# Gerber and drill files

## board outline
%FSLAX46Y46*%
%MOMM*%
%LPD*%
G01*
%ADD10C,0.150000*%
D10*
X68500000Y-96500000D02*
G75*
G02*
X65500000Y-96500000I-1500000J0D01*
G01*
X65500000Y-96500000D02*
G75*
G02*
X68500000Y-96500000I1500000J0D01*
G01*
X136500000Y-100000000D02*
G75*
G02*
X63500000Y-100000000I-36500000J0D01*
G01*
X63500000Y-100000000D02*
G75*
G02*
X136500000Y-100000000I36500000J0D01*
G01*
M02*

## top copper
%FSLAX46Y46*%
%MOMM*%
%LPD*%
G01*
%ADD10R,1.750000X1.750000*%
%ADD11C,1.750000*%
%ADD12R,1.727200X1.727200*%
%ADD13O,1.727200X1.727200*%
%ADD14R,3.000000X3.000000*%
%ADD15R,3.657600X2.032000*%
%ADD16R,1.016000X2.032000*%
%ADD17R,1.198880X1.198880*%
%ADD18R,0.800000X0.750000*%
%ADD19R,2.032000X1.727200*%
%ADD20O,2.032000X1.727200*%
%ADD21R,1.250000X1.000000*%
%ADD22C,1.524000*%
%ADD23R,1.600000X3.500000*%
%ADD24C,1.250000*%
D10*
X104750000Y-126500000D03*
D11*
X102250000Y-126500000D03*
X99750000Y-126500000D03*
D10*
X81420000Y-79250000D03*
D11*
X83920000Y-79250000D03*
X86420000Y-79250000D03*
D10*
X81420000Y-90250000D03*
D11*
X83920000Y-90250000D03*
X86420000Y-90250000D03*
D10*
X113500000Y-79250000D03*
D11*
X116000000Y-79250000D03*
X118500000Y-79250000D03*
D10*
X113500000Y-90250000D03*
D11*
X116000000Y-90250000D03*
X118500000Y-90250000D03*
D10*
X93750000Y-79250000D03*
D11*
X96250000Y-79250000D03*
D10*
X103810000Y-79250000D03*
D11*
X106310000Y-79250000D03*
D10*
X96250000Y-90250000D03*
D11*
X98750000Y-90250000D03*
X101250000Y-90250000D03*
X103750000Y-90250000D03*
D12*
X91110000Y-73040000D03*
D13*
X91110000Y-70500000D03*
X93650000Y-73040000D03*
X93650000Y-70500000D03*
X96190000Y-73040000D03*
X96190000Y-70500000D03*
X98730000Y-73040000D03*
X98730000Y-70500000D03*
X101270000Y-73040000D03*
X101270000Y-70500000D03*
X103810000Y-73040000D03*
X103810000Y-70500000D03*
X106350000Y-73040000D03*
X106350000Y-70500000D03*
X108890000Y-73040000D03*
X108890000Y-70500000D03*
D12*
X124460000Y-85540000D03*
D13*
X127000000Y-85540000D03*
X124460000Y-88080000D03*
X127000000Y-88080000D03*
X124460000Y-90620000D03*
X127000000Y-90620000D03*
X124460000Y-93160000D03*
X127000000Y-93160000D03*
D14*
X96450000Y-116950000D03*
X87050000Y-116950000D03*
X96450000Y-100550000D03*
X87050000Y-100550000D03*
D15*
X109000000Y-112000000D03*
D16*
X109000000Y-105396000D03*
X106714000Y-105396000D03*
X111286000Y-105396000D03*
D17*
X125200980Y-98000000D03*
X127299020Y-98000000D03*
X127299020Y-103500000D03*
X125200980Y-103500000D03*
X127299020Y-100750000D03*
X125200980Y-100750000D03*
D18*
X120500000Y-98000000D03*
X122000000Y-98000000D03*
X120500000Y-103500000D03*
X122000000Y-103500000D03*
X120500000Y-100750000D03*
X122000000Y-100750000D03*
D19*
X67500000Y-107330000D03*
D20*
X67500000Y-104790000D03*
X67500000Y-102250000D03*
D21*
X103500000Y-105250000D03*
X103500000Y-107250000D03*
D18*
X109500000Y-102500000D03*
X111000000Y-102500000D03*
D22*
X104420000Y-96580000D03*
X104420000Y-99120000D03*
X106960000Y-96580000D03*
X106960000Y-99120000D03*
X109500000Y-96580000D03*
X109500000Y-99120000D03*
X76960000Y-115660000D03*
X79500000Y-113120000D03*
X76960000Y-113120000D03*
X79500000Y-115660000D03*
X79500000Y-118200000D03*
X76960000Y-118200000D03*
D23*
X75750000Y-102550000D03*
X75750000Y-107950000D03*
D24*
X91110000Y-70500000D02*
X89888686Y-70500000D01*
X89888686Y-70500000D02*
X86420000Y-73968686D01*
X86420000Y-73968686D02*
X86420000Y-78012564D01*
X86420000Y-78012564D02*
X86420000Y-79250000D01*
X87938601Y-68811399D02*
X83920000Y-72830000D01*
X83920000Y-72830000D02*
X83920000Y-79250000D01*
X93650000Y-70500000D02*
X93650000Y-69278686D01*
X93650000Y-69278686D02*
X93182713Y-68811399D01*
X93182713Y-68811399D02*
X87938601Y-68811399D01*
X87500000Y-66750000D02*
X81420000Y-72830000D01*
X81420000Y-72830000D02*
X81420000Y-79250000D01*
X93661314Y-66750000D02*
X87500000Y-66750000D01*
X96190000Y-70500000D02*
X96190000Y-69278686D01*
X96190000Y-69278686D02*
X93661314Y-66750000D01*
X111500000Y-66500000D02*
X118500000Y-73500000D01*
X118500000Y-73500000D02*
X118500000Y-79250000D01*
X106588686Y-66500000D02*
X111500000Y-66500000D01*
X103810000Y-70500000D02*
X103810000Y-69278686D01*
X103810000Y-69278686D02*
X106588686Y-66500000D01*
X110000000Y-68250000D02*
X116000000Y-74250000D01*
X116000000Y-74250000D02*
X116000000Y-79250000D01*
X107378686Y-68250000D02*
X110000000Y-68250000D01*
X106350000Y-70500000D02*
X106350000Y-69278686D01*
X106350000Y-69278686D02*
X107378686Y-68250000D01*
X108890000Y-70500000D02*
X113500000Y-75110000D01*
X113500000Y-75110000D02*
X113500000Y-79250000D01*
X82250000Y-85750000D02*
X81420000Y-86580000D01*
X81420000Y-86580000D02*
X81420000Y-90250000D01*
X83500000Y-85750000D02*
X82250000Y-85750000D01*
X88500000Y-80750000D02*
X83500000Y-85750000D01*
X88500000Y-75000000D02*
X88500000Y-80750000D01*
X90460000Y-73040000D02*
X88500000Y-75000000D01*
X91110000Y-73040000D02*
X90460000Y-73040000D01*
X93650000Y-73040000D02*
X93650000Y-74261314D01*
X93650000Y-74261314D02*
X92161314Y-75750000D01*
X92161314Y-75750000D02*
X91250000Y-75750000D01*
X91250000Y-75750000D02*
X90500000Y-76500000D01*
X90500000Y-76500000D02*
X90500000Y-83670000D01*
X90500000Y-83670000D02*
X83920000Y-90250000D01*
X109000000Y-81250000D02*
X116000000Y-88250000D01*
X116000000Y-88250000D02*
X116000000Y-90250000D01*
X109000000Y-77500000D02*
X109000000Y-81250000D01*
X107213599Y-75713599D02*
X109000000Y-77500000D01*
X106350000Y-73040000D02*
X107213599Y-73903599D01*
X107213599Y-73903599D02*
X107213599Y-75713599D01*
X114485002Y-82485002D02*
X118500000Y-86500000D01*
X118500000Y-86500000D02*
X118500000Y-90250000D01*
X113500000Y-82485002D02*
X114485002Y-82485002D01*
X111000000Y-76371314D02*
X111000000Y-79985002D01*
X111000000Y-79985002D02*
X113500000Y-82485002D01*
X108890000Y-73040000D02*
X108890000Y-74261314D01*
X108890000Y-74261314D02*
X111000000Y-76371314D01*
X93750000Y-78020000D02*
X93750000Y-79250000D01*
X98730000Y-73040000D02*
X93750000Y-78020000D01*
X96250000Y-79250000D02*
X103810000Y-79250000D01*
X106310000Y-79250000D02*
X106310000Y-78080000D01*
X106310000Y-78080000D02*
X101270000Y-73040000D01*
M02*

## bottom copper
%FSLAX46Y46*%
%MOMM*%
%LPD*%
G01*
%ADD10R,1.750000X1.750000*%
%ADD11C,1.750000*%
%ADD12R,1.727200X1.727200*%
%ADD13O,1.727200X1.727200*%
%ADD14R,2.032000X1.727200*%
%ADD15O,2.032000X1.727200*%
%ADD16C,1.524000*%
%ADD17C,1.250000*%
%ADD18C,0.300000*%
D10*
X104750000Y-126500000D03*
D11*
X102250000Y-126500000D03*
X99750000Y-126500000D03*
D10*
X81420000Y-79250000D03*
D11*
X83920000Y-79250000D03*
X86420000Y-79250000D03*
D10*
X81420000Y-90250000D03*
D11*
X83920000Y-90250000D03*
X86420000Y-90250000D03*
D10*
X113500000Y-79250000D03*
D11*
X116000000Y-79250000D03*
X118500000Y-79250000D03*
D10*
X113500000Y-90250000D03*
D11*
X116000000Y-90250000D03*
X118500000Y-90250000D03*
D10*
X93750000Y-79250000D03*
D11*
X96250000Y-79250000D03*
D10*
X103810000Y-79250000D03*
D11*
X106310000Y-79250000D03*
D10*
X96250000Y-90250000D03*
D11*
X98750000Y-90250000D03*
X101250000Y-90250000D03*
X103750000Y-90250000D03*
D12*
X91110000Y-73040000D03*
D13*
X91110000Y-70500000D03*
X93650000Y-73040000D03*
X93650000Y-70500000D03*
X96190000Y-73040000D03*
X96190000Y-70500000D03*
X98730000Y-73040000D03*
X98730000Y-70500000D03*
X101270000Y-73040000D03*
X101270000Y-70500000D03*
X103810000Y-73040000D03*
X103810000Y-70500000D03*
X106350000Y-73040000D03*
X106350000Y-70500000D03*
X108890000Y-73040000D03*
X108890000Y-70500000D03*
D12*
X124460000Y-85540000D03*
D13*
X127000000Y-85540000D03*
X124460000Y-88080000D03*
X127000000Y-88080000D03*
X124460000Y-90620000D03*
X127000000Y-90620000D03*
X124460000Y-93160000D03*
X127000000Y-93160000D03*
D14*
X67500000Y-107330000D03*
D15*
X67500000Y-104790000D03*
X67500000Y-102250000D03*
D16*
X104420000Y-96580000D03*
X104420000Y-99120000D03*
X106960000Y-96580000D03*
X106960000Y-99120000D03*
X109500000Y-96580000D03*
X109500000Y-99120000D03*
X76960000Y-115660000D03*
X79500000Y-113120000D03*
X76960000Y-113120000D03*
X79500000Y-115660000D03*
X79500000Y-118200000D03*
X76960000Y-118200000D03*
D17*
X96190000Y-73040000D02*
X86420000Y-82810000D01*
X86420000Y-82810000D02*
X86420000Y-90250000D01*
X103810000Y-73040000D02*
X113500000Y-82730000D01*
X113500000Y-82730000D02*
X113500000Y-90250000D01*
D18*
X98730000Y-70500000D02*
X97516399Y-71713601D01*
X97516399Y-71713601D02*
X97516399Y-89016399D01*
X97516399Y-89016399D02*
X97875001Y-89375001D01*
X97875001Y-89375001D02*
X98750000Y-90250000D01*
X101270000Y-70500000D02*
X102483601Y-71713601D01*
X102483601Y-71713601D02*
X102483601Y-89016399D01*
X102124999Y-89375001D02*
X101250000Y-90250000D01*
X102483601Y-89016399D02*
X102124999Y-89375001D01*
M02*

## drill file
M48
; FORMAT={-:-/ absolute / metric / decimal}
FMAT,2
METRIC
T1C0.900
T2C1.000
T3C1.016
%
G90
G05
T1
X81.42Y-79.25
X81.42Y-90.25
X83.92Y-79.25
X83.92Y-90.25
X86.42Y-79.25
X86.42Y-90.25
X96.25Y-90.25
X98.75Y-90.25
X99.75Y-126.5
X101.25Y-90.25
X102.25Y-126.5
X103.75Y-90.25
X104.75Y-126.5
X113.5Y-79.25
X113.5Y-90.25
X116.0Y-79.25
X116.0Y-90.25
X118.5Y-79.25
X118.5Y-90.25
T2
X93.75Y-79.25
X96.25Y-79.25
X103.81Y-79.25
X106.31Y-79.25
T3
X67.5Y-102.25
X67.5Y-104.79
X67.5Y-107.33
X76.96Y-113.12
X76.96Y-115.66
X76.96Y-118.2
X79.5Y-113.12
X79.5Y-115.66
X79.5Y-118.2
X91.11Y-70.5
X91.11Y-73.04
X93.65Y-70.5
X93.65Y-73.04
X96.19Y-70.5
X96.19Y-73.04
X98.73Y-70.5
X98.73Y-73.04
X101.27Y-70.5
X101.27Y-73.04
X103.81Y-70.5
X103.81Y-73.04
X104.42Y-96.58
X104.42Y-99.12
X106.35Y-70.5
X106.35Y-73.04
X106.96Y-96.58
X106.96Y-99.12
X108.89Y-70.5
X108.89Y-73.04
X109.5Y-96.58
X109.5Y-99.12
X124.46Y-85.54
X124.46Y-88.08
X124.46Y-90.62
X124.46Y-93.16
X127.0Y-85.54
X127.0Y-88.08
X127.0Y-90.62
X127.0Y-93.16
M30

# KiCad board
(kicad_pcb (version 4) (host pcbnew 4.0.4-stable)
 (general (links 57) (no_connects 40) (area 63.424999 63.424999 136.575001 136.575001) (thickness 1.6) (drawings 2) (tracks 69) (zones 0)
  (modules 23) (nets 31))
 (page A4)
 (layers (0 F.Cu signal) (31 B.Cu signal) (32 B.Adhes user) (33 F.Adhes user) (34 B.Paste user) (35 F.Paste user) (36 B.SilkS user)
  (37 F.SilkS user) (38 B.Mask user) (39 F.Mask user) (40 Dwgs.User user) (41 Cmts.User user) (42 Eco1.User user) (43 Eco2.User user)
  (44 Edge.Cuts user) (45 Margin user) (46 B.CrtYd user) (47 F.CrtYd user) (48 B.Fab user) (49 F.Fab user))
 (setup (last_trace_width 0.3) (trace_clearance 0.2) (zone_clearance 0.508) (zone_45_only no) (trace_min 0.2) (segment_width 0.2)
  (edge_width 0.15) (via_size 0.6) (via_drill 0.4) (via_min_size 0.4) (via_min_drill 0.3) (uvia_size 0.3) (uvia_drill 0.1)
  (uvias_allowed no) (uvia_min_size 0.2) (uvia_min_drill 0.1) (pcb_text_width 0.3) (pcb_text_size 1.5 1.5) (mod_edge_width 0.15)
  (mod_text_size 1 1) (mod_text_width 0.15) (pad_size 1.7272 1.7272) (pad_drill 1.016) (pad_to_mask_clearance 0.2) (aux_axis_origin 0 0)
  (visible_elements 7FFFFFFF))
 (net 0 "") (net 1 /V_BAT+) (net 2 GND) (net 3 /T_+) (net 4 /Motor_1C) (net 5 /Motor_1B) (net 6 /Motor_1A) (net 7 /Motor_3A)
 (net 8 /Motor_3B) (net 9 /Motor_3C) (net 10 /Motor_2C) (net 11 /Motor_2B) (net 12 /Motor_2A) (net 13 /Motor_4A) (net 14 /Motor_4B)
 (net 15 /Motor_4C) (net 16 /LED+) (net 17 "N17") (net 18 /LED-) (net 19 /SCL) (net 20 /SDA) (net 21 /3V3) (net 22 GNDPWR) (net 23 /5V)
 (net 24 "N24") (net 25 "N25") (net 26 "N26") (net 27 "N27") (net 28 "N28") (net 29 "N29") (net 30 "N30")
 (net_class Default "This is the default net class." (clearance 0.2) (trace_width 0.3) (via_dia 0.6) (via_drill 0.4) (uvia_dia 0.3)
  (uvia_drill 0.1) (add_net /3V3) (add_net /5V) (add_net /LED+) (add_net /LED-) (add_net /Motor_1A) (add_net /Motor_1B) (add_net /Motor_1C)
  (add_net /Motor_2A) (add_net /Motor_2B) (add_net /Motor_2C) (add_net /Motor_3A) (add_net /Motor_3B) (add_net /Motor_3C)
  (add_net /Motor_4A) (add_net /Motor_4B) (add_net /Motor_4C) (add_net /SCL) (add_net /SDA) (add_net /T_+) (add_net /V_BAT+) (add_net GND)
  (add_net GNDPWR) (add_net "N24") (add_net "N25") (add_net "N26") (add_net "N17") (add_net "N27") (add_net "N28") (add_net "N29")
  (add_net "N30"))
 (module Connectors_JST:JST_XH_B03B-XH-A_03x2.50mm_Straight (layer F.Cu) (at 104.75 126.5 180)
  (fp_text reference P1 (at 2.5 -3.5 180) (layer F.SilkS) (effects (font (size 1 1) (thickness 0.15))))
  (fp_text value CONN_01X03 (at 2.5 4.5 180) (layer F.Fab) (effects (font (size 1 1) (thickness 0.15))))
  (pad 1 thru_hole rect (at 0 0 180) (size 1.75 1.75) (drill 0.9) (layers *.Cu *.Mask) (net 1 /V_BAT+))
  (pad 2 thru_hole circle (at 2.5 0 180) (size 1.75 1.75) (drill 0.9) (layers *.Cu *.Mask) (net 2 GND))
  (pad 3 thru_hole circle (at 5 0 180) (size 1.75 1.75) (drill 0.9) (layers *.Cu *.Mask) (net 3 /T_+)))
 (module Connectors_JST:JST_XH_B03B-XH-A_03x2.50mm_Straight (layer F.Cu) (at 81.42 79.25)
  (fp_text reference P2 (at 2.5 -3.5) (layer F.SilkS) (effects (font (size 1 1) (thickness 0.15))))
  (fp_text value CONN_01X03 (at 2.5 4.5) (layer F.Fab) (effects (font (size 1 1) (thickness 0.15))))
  (pad 1 thru_hole rect (at 0 0) (size 1.75 1.75) (drill 0.9) (layers *.Cu *.Mask) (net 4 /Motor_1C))
  (pad 2 thru_hole circle (at 2.5 0) (size 1.75 1.75) (drill 0.9) (layers *.Cu *.Mask) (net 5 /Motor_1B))
  (pad 3 thru_hole circle (at 5 0) (size 1.75 1.75) (drill 0.9) (layers *.Cu *.Mask) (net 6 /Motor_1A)))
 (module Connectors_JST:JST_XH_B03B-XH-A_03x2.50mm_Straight (layer F.Cu) (at 81.42 90.25)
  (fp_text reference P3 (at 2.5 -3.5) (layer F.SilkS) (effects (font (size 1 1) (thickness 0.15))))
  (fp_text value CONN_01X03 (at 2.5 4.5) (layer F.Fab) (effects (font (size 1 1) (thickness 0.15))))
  (pad 1 thru_hole rect (at 0 0) (size 1.75 1.75) (drill 0.9) (layers *.Cu *.Mask) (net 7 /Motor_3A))
  (pad 2 thru_hole circle (at 2.5 0) (size 1.75 1.75) (drill 0.9) (layers *.Cu *.Mask) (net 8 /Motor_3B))
  (pad 3 thru_hole circle (at 5 0) (size 1.75 1.75) (drill 0.9) (layers *.Cu *.Mask) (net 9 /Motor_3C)))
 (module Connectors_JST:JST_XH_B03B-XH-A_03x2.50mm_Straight (layer F.Cu) (at 113.5 79.25)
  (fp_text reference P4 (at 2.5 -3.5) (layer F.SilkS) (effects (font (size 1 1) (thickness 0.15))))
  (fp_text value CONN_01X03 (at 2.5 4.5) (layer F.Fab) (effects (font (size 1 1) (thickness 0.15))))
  (pad 1 thru_hole rect (at 0 0) (size 1.75 1.75) (drill 0.9) (layers *.Cu *.Mask) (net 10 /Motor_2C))
  (pad 2 thru_hole circle (at 2.5 0) (size 1.75 1.75) (drill 0.9) (layers *.Cu *.Mask) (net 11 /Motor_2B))
  (pad 3 thru_hole circle (at 5 0) (size 1.75 1.75) (drill 0.9) (layers *.Cu *.Mask) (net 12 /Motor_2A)))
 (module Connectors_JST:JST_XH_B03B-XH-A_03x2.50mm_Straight (layer F.Cu) (at 113.5 90.25)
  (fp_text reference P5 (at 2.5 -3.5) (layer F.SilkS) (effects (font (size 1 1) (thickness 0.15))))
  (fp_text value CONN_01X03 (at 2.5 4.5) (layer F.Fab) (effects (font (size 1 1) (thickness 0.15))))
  (pad 1 thru_hole rect (at 0 0) (size 1.75 1.75) (drill 0.9) (layers *.Cu *.Mask) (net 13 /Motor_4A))
  (pad 2 thru_hole circle (at 2.5 0) (size 1.75 1.75) (drill 0.9) (layers *.Cu *.Mask) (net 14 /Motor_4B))
  (pad 3 thru_hole circle (at 5 0) (size 1.75 1.75) (drill 0.9) (layers *.Cu *.Mask) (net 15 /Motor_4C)))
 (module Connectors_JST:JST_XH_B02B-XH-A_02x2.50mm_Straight (layer F.Cu) (at 93.75 79.25)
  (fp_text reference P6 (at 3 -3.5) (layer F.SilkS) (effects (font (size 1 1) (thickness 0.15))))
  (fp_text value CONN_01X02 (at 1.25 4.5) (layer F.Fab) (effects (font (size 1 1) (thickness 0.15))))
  (pad 1 thru_hole rect (at 0 0) (size 1.75 1.75) (drill 1) (layers *.Cu *.Mask) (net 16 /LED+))
  (pad 2 thru_hole circle (at 2.5 0) (size 1.75 1.75) (drill 1) (layers *.Cu *.Mask) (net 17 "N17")))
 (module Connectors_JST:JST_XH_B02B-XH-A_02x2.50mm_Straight (layer F.Cu) (at 103.81 79.25)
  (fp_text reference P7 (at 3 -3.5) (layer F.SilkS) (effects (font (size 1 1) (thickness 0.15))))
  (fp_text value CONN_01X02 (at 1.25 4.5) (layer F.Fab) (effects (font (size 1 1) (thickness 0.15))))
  (pad 1 thru_hole rect (at 0 0) (size 1.75 1.75) (drill 1) (layers *.Cu *.Mask) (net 17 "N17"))
  (pad 2 thru_hole circle (at 2.5 0) (size 1.75 1.75) (drill 1) (layers *.Cu *.Mask) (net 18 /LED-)))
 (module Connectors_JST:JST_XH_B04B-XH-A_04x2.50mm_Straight (layer F.Cu) (at 96.25 90.25)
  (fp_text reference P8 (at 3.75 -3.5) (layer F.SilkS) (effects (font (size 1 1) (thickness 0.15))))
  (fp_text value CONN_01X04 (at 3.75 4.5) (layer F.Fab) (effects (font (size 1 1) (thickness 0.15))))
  (pad 1 thru_hole rect (at 0 0) (size 1.75 1.75) (drill 0.9) (layers *.Cu *.Mask) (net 2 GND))
  (pad 2 thru_hole circle (at 2.5 0) (size 1.75 1.75) (drill 0.9) (layers *.Cu *.Mask) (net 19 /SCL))
  (pad 3 thru_hole circle (at 5 0) (size 1.75 1.75) (drill 0.9) (layers *.Cu *.Mask) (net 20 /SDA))
  (pad 4 thru_hole circle (at 7.5 0) (size 1.75 1.75) (drill 0.9) (layers *.Cu *.Mask) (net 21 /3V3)))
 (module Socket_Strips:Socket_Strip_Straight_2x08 (layer B.Cu) (at 91.11 73.04)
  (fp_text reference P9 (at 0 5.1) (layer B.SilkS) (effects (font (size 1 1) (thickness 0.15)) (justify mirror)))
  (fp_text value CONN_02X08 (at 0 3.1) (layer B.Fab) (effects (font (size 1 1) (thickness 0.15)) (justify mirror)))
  (pad 1 thru_hole rect (at 0 0) (size 1.7272 1.7272) (drill 1.016) (layers *.Cu *.Mask B.SilkS) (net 7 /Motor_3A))
  (pad 2 thru_hole oval (at 0 -2.54) (size 1.7272 1.7272) (drill 1.016) (layers *.Cu *.Mask B.SilkS) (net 6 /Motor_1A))
  (pad 3 thru_hole oval (at 2.54 0) (size 1.7272 1.7272) (drill 1.016) (layers *.Cu *.Mask B.SilkS) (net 8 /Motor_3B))
  (pad 4 thru_hole oval (at 2.54 -2.54) (size 1.7272 1.7272) (drill 1.016) (layers *.Cu *.Mask B.SilkS) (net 5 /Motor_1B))
  (pad 5 thru_hole oval (at 5.08 0) (size 1.7272 1.7272) (drill 1.016) (layers *.Cu *.Mask B.SilkS) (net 9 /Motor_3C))
  (pad 6 thru_hole oval (at 5.08 -2.54) (size 1.7272 1.7272) (drill 1.016) (layers *.Cu *.Mask B.SilkS) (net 4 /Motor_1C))
  (pad 7 thru_hole oval (at 7.62 0) (size 1.7272 1.7272) (drill 1.016) (layers *.Cu *.Mask B.SilkS) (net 16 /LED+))
  (pad 8 thru_hole oval (at 7.62 -2.54) (size 1.7272 1.7272) (drill 1.016) (layers *.Cu *.Mask B.SilkS) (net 19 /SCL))
  (pad 9 thru_hole oval (at 10.16 0) (size 1.7272 1.7272) (drill 1.016) (layers *.Cu *.Mask B.SilkS) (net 18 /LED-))
  (pad 10 thru_hole oval (at 10.16 -2.54) (size 1.7272 1.7272) (drill 1.016) (layers *.Cu *.Mask B.SilkS) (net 20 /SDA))
  (pad 11 thru_hole oval (at 12.7 0) (size 1.7272 1.7272) (drill 1.016) (layers *.Cu *.Mask B.SilkS) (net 13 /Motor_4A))
  (pad 12 thru_hole oval (at 12.7 -2.54) (size 1.7272 1.7272) (drill 1.016) (layers *.Cu *.Mask B.SilkS) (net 12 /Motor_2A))
  (pad 13 thru_hole oval (at 15.24 0) (size 1.7272 1.7272) (drill 1.016) (layers *.Cu *.Mask B.SilkS) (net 14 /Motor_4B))
  (pad 14 thru_hole oval (at 15.24 -2.54) (size 1.7272 1.7272) (drill 1.016) (layers *.Cu *.Mask B.SilkS) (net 11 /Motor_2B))
  (pad 15 thru_hole oval (at 17.78 0) (size 1.7272 1.7272) (drill 1.016) (layers *.Cu *.Mask B.SilkS) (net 15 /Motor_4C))
  (pad 16 thru_hole oval (at 17.78 -2.54) (size 1.7272 1.7272) (drill 1.016) (layers *.Cu *.Mask B.SilkS) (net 10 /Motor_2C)))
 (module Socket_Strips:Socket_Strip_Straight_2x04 (layer B.Cu) (at 124.46 85.54 270)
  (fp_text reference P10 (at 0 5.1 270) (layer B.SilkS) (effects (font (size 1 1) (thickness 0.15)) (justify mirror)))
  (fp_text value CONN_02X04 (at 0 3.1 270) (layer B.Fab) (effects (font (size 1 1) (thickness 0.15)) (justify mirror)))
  (pad 1 thru_hole rect (at 0 0 270) (size 1.7272 1.7272) (drill 1.016) (layers *.Cu *.Mask B.SilkS) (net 1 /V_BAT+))
  (pad 2 thru_hole oval (at 0 -2.54 270) (size 1.7272 1.7272) (drill 1.016) (layers *.Cu *.Mask B.SilkS) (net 1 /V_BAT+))
  (pad 3 thru_hole oval (at 2.54 0 270) (size 1.7272 1.7272) (drill 1.016) (layers *.Cu *.Mask B.SilkS) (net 1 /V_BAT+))
  (pad 4 thru_hole oval (at 2.54 -2.54 270) (size 1.7272 1.7272) (drill 1.016) (layers *.Cu *.Mask B.SilkS) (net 1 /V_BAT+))
  (pad 5 thru_hole oval (at 5.08 0 270) (size 1.7272 1.7272) (drill 1.016) (layers *.Cu *.Mask B.SilkS) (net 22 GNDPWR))
  (pad 6 thru_hole oval (at 5.08 -2.54 270) (size 1.7272 1.7272) (drill 1.016) (layers *.Cu *.Mask B.SilkS) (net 22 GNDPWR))
  (pad 7 thru_hole oval (at 7.62 0 270) (size 1.7272 1.7272) (drill 1.016) (layers *.Cu *.Mask B.SilkS) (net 22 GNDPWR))
  (pad 8 thru_hole oval (at 7.62 -2.54 270) (size 1.7272 1.7272) (drill 1.016) (layers *.Cu *.Mask B.SilkS) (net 22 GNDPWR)))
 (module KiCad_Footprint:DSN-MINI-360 (layer F.Cu) (at 91.75 108.75 270)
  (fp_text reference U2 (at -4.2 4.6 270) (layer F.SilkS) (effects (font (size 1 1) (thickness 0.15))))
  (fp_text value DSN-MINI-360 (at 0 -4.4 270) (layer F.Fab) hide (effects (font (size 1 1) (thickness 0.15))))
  (pad 1 smd rect (at 8.2 -4.7 270) (size 3 3) (layers F.Cu F.Paste F.Mask) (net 1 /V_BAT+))
  (pad 2 smd rect (at 8.2 4.7 270) (size 3 3) (layers F.Cu F.Paste F.Mask) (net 22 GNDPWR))
  (pad 3 smd rect (at -8.2 -4.7 270) (size 3 3) (layers F.Cu F.Paste F.Mask) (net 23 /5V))
  (pad 4 smd rect (at -8.2 4.7 270) (size 3 3) (layers F.Cu F.Paste F.Mask) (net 2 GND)))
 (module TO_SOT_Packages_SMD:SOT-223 (layer F.Cu) (at 109 108.698 180)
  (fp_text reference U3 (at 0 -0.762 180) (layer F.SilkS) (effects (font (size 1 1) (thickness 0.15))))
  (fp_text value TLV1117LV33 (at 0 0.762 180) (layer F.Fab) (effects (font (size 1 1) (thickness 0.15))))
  (pad 4 smd rect (at 0 -3.302 180) (size 3.6576 2.032) (layers F.Cu F.Paste F.Mask) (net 21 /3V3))
  (pad 2 smd rect (at 0 3.302 180) (size 1.016 2.032) (layers F.Cu F.Paste F.Mask) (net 21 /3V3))
  (pad 3 smd rect (at 2.286 3.302 180) (size 1.016 2.032) (layers F.Cu F.Paste F.Mask) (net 23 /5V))
  (pad 1 smd rect (at -2.286 3.302 180) (size 1.016 2.032) (layers F.Cu F.Paste F.Mask) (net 2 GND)))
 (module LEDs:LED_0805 (layer F.Cu) (at 126.25 98 180)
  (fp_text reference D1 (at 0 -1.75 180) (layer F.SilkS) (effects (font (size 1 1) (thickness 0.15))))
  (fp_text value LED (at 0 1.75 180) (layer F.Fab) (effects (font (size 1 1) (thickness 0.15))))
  (pad 2 smd rect (at 1.04902 0) (size 1.19888 1.19888) (layers F.Cu F.Paste F.Mask) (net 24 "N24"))
  (pad 1 smd rect (at -1.04902 0) (size 1.19888 1.19888) (layers F.Cu F.Paste F.Mask) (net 2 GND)))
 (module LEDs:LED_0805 (layer F.Cu) (at 126.25 103.5)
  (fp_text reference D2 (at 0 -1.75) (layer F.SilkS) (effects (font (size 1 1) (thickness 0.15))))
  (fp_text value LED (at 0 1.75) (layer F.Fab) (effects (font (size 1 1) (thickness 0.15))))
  (pad 2 smd rect (at 1.04902 0 180) (size 1.19888 1.19888) (layers F.Cu F.Paste F.Mask) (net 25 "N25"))
  (pad 1 smd rect (at -1.04902 0 180) (size 1.19888 1.19888) (layers F.Cu F.Paste F.Mask) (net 2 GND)))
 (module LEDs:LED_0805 (layer F.Cu) (at 126.25 100.75)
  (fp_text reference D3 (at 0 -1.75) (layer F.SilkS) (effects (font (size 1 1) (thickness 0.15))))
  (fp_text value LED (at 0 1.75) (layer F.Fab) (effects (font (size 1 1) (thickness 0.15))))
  (pad 2 smd rect (at 1.04902 0 180) (size 1.19888 1.19888) (layers F.Cu F.Paste F.Mask) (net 21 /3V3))
  (pad 1 smd rect (at -1.04902 0 180) (size 1.19888 1.19888) (layers F.Cu F.Paste F.Mask) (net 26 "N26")))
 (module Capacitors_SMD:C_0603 (layer F.Cu) (at 121.25 98)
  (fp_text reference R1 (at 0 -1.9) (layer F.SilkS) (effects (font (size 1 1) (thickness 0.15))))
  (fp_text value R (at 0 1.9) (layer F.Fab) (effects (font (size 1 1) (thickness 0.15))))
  (pad 1 smd rect (at -0.75 0) (size 0.8 0.75) (layers F.Cu F.Paste F.Mask) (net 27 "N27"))
  (pad 2 smd rect (at 0.75 0) (size 0.8 0.75) (layers F.Cu F.Paste F.Mask) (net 24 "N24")))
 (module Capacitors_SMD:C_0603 (layer F.Cu) (at 121.25 103.5)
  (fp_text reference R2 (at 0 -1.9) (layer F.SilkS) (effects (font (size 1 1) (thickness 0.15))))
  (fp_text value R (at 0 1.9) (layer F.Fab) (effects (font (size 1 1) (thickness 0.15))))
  (pad 1 smd rect (at -0.75 0) (size 0.8 0.75) (layers F.Cu F.Paste F.Mask) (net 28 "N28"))
  (pad 2 smd rect (at 0.75 0) (size 0.8 0.75) (layers F.Cu F.Paste F.Mask) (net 25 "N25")))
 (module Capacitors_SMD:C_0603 (layer F.Cu) (at 121.25 100.75)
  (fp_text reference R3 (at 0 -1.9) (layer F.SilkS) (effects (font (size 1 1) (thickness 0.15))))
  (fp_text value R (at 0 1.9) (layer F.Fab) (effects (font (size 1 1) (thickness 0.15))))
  (pad 1 smd rect (at -0.75 0) (size 0.8 0.75) (layers F.Cu F.Paste F.Mask) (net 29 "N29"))
  (pad 2 smd rect (at 0.75 0) (size 0.8 0.75) (layers F.Cu F.Paste F.Mask) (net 26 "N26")))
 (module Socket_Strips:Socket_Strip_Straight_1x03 (layer B.Cu) (at 67.5 107.33 90)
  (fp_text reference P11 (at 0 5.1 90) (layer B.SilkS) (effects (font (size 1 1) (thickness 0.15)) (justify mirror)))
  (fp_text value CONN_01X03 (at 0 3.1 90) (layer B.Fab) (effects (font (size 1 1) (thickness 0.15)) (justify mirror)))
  (pad 1 thru_hole rect (at 0 0 90) (size 1.7272 2.032) (drill 1.016) (layers *.Cu *.Mask B.SilkS) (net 2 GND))
  (pad 2 thru_hole oval (at 2.54 0 90) (size 1.7272 2.032) (drill 1.016) (layers *.Cu *.Mask B.SilkS))
  (pad 3 thru_hole oval (at 5.08 0 90) (size 1.7272 2.032) (drill 1.016) (layers *.Cu *.Mask B.SilkS) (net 23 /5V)))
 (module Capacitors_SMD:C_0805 (layer F.Cu) (at 103.5 106.25 270)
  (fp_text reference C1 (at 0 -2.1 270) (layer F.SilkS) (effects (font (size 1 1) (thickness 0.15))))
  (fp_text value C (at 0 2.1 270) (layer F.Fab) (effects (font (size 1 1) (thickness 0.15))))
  (pad 1 smd rect (at -1 0 270) (size 1 1.25) (layers F.Cu F.Paste F.Mask) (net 23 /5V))
  (pad 2 smd rect (at 1 0 270) (size 1 1.25) (layers F.Cu F.Paste F.Mask) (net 2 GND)))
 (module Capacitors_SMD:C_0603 (layer F.Cu) (at 110.25 102.5)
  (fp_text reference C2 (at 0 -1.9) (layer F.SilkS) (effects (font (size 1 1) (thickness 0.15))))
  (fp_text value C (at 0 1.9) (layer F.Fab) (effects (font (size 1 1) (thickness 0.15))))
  (pad 1 smd rect (at -0.75 0) (size 0.8 0.75) (layers F.Cu F.Paste F.Mask) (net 21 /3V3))
  (pad 2 smd rect (at 0.75 0) (size 0.8 0.75) (layers F.Cu F.Paste F.Mask) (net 2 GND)))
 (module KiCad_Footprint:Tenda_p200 (layer B.Cu) (at 93.32 100)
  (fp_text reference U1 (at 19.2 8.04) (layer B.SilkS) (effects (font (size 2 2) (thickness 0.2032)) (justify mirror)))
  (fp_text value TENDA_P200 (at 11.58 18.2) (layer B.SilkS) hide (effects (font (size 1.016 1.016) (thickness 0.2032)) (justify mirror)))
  (pad 3V3 thru_hole circle (at 11.1 -3.42) (size 1.524 1.524) (drill 1.016) (layers *.Cu *.Mask B.SilkS) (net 21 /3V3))
  (pad 3V3 thru_hole circle (at 11.1 -0.88) (size 1.524 1.524) (drill 1.016) (layers *.Cu *.Mask B.SilkS) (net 21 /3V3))
  (pad C thru_hole circle (at 13.64 -3.42) (size 1.524 1.524) (drill 1.016) (layers *.Cu *.Mask B.SilkS) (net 28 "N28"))
  (pad P thru_hole circle (at 13.64 -0.88) (size 1.524 1.524) (drill 1.016) (layers *.Cu *.Mask B.SilkS) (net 27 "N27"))
  (pad E thru_hole circle (at 16.18 -3.42) (size 1.524 1.524) (drill 1.016) (layers *.Cu *.Mask B.SilkS) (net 29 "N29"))
  (pad GND thru_hole circle (at 16.18 -0.88) (size 1.524 1.524) (drill 1.016) (layers *.Cu *.Mask B.SilkS) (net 2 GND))
  (pad NC thru_hole circle (at -16.36 15.66 270) (size 1.524 1.524) (drill 1.016) (layers *.Cu *.Mask B.SilkS) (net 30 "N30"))
  (pad T_+ thru_hole circle (at -13.82 13.12 270) (size 1.524 1.524) (drill 1.016) (layers *.Cu *.Mask B.SilkS) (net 3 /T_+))
  (pad T_+ thru_hole circle (at -16.36 13.12 270) (size 1.524 1.524) (drill 1.016) (layers *.Cu *.Mask B.SilkS) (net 3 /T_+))
  (pad NC thru_hole circle (at -13.82 15.66 270) (size 1.524 1.524) (drill 1.016) (layers *.Cu *.Mask B.SilkS) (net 30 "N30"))
  (pad T_- thru_hole circle (at -13.82 18.2 270) (size 1.524 1.524) (drill 1.016) (layers *.Cu *.Mask B.SilkS) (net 22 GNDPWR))
  (pad T_- thru_hole circle (at -16.36 18.2 270) (size 1.524 1.524) (drill 1.016) (layers *.Cu *.Mask B.SilkS) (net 22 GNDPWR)))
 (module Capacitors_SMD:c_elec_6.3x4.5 (layer F.Cu) (at 75.75 105.25 270)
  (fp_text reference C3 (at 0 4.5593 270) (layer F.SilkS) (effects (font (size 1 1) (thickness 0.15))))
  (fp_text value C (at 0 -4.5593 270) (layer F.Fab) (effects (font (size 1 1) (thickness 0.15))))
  (pad 1 smd rect (at -2.7 0 90) (size 3.5 1.6) (layers F.Cu F.Paste F.Mask) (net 23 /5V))
  (pad 2 smd rect (at 2.7 0 90) (size 3.5 1.6) (layers F.Cu F.Paste F.Mask) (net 2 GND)))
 (gr_circle (center 67 96.5) (end 67 98) (layer Edge.Cuts) (width 0.15))
 (gr_circle (center 100 100) (end 100 136.5) (layer Edge.Cuts) (width 0.15))
 (segment (start 91.11 70.5) (end 89.888686 70.5) (width 1.25) (layer F.Cu) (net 6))
 (segment (start 89.888686 70.5) (end 86.42 73.968686) (width 1.25) (layer F.Cu) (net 6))
 (segment (start 86.42 73.968686) (end 86.42 78.012564) (width 1.25) (layer F.Cu) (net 6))
 (segment (start 86.42 78.012564) (end 86.42 79.25) (width 1.25) (layer F.Cu) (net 6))
 (segment (start 87.938601 68.811399) (end 83.92 72.83) (width 1.25) (layer F.Cu) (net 5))
 (segment (start 83.92 72.83) (end 83.92 79.25) (width 1.25) (layer F.Cu) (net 5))
 (segment (start 93.65 70.5) (end 93.65 69.278686) (width 1.25) (layer F.Cu) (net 5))
 (segment (start 93.65 69.278686) (end 93.182713 68.811399) (width 1.25) (layer F.Cu) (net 5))
 (segment (start 93.182713 68.811399) (end 87.938601 68.811399) (width 1.25) (layer F.Cu) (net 5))
 (segment (start 87.5 66.75) (end 81.42 72.83) (width 1.25) (layer F.Cu) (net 4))
 (segment (start 81.42 72.83) (end 81.42 79.25) (width 1.25) (layer F.Cu) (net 4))
 (segment (start 93.661314 66.75) (end 87.5 66.75) (width 1.25) (layer F.Cu) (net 4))
 (segment (start 96.19 70.5) (end 96.19 69.278686) (width 1.25) (layer F.Cu) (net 4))
 (segment (start 96.19 69.278686) (end 93.661314 66.75) (width 1.25) (layer F.Cu) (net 4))
 (segment (start 111.5 66.5) (end 118.5 73.5) (width 1.25) (layer F.Cu) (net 12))
 (segment (start 118.5 73.5) (end 118.5 79.25) (width 1.25) (layer F.Cu) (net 12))
 (segment (start 106.588686 66.5) (end 111.5 66.5) (width 1.25) (layer F.Cu) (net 12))
 (segment (start 103.81 70.5) (end 103.81 69.278686) (width 1.25) (layer F.Cu) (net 12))
 (segment (start 103.81 69.278686) (end 106.588686 66.5) (width 1.25) (layer F.Cu) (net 12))
 (segment (start 110 68.25) (end 116 74.25) (width 1.25) (layer F.Cu) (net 11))
 (segment (start 116 74.25) (end 116 79.25) (width 1.25) (layer F.Cu) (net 11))
 (segment (start 107.378686 68.25) (end 110 68.25) (width 1.25) (layer F.Cu) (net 11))
 (segment (start 106.35 70.5) (end 106.35 69.278686) (width 1.25) (layer F.Cu) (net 11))
 (segment (start 106.35 69.278686) (end 107.378686 68.25) (width 1.25) (layer F.Cu) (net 11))
 (segment (start 108.89 70.5) (end 113.5 75.11) (width 1.25) (layer F.Cu) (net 10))
 (segment (start 113.5 75.11) (end 113.5 79.25) (width 1.25) (layer F.Cu) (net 10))
 (segment (start 82.25 85.75) (end 81.42 86.58) (width 1.25) (layer F.Cu) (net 7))
 (segment (start 81.42 86.58) (end 81.42 90.25) (width 1.25) (layer F.Cu) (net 7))
 (segment (start 83.5 85.75) (end 82.25 85.75) (width 1.25) (layer F.Cu) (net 7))
 (segment (start 88.5 80.75) (end 83.5 85.75) (width 1.25) (layer F.Cu) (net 7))
 (segment (start 88.5 75) (end 88.5 80.75) (width 1.25) (layer F.Cu) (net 7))
 (segment (start 90.46 73.04) (end 88.5 75) (width 1.25) (layer F.Cu) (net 7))
 (segment (start 91.11 73.04) (end 90.46 73.04) (width 1.25) (layer F.Cu) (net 7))
 (segment (start 93.65 73.04) (end 93.65 74.261314) (width 1.25) (layer F.Cu) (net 8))
 (segment (start 93.65 74.261314) (end 92.161314 75.75) (width 1.25) (layer F.Cu) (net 8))
 (segment (start 92.161314 75.75) (end 91.25 75.75) (width 1.25) (layer F.Cu) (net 8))
 (segment (start 91.25 75.75) (end 90.5 76.5) (width 1.25) (layer F.Cu) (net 8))
 (segment (start 90.5 76.5) (end 90.5 83.67) (width 1.25) (layer F.Cu) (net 8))
 (segment (start 90.5 83.67) (end 83.92 90.25) (width 1.25) (layer F.Cu) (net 8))
 (segment (start 96.19 73.04) (end 86.42 82.81) (width 1.25) (layer B.Cu) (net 9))
 (segment (start 86.42 82.81) (end 86.42 90.25) (width 1.25) (layer B.Cu) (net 9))
 (segment (start 103.81 73.04) (end 113.5 82.73) (width 1.25) (layer B.Cu) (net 13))
 (segment (start 113.5 82.73) (end 113.5 90.25) (width 1.25) (layer B.Cu) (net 13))
 (segment (start 109 81.25) (end 116 88.25) (width 1.25) (layer F.Cu) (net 14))
 (segment (start 116 88.25) (end 116 90.25) (width 1.25) (layer F.Cu) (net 14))
 (segment (start 109 77.5) (end 109 81.25) (width 1.25) (layer F.Cu) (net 14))
 (segment (start 107.213599 75.713599) (end 109 77.5) (width 1.25) (layer F.Cu) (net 14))
 (segment (start 106.35 73.04) (end 107.213599 73.903599) (width 1.25) (layer F.Cu) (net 14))
 (segment (start 107.213599 73.903599) (end 107.213599 75.713599) (width 1.25) (layer F.Cu) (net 14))
 (segment (start 114.485002 82.485002) (end 118.5 86.5) (width 1.25) (layer F.Cu) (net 15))
 (segment (start 118.5 86.5) (end 118.5 90.25) (width 1.25) (layer F.Cu) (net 15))
 (segment (start 113.5 82.485002) (end 114.485002 82.485002) (width 1.25) (layer F.Cu) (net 15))
 (segment (start 111 76.371314) (end 111 79.985002) (width 1.25) (layer F.Cu) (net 15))
 (segment (start 111 79.985002) (end 113.5 82.485002) (width 1.25) (layer F.Cu) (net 15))
 (segment (start 108.89 73.04) (end 108.89 74.261314) (width 1.25) (layer F.Cu) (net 15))
 (segment (start 108.89 74.261314) (end 111 76.371314) (width 1.25) (layer F.Cu) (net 15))
 (segment (start 93.75 78.02) (end 93.75 79.25) (width 1.25) (layer F.Cu) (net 16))
 (segment (start 98.73 73.04) (end 93.75 78.02) (width 1.25) (layer F.Cu) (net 16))
 (segment (start 96.25 79.25) (end 103.81 79.25) (width 1.25) (layer F.Cu) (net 17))
 (segment (start 106.31 79.25) (end 106.31 78.08) (width 1.25) (layer F.Cu) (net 18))
 (segment (start 106.31 78.08) (end 101.27 73.04) (width 1.25) (layer F.Cu) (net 18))
 (segment (start 98.73 70.5) (end 97.516399 71.713601) (width 0.3) (layer B.Cu) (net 19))
 (segment (start 97.516399 71.713601) (end 97.516399 89.016399) (width 0.3) (layer B.Cu) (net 19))
 (segment (start 97.516399 89.016399) (end 97.875001 89.375001) (width 0.3) (layer B.Cu) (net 19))
 (segment (start 97.875001 89.375001) (end 98.75 90.25) (width 0.3) (layer B.Cu) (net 19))
 (segment (start 101.27 70.5) (end 102.483601 71.713601) (width 0.3) (layer B.Cu) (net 20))
 (segment (start 102.483601 71.713601) (end 102.483601 89.016399) (width 0.3) (layer B.Cu) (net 20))
 (segment (start 102.124999 89.375001) (end 101.25 90.25) (width 0.3) (layer B.Cu) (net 20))
 (segment (start 102.483601 89.016399) (end 102.124999 89.375001) (width 0.3) (layer B.Cu) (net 20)))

